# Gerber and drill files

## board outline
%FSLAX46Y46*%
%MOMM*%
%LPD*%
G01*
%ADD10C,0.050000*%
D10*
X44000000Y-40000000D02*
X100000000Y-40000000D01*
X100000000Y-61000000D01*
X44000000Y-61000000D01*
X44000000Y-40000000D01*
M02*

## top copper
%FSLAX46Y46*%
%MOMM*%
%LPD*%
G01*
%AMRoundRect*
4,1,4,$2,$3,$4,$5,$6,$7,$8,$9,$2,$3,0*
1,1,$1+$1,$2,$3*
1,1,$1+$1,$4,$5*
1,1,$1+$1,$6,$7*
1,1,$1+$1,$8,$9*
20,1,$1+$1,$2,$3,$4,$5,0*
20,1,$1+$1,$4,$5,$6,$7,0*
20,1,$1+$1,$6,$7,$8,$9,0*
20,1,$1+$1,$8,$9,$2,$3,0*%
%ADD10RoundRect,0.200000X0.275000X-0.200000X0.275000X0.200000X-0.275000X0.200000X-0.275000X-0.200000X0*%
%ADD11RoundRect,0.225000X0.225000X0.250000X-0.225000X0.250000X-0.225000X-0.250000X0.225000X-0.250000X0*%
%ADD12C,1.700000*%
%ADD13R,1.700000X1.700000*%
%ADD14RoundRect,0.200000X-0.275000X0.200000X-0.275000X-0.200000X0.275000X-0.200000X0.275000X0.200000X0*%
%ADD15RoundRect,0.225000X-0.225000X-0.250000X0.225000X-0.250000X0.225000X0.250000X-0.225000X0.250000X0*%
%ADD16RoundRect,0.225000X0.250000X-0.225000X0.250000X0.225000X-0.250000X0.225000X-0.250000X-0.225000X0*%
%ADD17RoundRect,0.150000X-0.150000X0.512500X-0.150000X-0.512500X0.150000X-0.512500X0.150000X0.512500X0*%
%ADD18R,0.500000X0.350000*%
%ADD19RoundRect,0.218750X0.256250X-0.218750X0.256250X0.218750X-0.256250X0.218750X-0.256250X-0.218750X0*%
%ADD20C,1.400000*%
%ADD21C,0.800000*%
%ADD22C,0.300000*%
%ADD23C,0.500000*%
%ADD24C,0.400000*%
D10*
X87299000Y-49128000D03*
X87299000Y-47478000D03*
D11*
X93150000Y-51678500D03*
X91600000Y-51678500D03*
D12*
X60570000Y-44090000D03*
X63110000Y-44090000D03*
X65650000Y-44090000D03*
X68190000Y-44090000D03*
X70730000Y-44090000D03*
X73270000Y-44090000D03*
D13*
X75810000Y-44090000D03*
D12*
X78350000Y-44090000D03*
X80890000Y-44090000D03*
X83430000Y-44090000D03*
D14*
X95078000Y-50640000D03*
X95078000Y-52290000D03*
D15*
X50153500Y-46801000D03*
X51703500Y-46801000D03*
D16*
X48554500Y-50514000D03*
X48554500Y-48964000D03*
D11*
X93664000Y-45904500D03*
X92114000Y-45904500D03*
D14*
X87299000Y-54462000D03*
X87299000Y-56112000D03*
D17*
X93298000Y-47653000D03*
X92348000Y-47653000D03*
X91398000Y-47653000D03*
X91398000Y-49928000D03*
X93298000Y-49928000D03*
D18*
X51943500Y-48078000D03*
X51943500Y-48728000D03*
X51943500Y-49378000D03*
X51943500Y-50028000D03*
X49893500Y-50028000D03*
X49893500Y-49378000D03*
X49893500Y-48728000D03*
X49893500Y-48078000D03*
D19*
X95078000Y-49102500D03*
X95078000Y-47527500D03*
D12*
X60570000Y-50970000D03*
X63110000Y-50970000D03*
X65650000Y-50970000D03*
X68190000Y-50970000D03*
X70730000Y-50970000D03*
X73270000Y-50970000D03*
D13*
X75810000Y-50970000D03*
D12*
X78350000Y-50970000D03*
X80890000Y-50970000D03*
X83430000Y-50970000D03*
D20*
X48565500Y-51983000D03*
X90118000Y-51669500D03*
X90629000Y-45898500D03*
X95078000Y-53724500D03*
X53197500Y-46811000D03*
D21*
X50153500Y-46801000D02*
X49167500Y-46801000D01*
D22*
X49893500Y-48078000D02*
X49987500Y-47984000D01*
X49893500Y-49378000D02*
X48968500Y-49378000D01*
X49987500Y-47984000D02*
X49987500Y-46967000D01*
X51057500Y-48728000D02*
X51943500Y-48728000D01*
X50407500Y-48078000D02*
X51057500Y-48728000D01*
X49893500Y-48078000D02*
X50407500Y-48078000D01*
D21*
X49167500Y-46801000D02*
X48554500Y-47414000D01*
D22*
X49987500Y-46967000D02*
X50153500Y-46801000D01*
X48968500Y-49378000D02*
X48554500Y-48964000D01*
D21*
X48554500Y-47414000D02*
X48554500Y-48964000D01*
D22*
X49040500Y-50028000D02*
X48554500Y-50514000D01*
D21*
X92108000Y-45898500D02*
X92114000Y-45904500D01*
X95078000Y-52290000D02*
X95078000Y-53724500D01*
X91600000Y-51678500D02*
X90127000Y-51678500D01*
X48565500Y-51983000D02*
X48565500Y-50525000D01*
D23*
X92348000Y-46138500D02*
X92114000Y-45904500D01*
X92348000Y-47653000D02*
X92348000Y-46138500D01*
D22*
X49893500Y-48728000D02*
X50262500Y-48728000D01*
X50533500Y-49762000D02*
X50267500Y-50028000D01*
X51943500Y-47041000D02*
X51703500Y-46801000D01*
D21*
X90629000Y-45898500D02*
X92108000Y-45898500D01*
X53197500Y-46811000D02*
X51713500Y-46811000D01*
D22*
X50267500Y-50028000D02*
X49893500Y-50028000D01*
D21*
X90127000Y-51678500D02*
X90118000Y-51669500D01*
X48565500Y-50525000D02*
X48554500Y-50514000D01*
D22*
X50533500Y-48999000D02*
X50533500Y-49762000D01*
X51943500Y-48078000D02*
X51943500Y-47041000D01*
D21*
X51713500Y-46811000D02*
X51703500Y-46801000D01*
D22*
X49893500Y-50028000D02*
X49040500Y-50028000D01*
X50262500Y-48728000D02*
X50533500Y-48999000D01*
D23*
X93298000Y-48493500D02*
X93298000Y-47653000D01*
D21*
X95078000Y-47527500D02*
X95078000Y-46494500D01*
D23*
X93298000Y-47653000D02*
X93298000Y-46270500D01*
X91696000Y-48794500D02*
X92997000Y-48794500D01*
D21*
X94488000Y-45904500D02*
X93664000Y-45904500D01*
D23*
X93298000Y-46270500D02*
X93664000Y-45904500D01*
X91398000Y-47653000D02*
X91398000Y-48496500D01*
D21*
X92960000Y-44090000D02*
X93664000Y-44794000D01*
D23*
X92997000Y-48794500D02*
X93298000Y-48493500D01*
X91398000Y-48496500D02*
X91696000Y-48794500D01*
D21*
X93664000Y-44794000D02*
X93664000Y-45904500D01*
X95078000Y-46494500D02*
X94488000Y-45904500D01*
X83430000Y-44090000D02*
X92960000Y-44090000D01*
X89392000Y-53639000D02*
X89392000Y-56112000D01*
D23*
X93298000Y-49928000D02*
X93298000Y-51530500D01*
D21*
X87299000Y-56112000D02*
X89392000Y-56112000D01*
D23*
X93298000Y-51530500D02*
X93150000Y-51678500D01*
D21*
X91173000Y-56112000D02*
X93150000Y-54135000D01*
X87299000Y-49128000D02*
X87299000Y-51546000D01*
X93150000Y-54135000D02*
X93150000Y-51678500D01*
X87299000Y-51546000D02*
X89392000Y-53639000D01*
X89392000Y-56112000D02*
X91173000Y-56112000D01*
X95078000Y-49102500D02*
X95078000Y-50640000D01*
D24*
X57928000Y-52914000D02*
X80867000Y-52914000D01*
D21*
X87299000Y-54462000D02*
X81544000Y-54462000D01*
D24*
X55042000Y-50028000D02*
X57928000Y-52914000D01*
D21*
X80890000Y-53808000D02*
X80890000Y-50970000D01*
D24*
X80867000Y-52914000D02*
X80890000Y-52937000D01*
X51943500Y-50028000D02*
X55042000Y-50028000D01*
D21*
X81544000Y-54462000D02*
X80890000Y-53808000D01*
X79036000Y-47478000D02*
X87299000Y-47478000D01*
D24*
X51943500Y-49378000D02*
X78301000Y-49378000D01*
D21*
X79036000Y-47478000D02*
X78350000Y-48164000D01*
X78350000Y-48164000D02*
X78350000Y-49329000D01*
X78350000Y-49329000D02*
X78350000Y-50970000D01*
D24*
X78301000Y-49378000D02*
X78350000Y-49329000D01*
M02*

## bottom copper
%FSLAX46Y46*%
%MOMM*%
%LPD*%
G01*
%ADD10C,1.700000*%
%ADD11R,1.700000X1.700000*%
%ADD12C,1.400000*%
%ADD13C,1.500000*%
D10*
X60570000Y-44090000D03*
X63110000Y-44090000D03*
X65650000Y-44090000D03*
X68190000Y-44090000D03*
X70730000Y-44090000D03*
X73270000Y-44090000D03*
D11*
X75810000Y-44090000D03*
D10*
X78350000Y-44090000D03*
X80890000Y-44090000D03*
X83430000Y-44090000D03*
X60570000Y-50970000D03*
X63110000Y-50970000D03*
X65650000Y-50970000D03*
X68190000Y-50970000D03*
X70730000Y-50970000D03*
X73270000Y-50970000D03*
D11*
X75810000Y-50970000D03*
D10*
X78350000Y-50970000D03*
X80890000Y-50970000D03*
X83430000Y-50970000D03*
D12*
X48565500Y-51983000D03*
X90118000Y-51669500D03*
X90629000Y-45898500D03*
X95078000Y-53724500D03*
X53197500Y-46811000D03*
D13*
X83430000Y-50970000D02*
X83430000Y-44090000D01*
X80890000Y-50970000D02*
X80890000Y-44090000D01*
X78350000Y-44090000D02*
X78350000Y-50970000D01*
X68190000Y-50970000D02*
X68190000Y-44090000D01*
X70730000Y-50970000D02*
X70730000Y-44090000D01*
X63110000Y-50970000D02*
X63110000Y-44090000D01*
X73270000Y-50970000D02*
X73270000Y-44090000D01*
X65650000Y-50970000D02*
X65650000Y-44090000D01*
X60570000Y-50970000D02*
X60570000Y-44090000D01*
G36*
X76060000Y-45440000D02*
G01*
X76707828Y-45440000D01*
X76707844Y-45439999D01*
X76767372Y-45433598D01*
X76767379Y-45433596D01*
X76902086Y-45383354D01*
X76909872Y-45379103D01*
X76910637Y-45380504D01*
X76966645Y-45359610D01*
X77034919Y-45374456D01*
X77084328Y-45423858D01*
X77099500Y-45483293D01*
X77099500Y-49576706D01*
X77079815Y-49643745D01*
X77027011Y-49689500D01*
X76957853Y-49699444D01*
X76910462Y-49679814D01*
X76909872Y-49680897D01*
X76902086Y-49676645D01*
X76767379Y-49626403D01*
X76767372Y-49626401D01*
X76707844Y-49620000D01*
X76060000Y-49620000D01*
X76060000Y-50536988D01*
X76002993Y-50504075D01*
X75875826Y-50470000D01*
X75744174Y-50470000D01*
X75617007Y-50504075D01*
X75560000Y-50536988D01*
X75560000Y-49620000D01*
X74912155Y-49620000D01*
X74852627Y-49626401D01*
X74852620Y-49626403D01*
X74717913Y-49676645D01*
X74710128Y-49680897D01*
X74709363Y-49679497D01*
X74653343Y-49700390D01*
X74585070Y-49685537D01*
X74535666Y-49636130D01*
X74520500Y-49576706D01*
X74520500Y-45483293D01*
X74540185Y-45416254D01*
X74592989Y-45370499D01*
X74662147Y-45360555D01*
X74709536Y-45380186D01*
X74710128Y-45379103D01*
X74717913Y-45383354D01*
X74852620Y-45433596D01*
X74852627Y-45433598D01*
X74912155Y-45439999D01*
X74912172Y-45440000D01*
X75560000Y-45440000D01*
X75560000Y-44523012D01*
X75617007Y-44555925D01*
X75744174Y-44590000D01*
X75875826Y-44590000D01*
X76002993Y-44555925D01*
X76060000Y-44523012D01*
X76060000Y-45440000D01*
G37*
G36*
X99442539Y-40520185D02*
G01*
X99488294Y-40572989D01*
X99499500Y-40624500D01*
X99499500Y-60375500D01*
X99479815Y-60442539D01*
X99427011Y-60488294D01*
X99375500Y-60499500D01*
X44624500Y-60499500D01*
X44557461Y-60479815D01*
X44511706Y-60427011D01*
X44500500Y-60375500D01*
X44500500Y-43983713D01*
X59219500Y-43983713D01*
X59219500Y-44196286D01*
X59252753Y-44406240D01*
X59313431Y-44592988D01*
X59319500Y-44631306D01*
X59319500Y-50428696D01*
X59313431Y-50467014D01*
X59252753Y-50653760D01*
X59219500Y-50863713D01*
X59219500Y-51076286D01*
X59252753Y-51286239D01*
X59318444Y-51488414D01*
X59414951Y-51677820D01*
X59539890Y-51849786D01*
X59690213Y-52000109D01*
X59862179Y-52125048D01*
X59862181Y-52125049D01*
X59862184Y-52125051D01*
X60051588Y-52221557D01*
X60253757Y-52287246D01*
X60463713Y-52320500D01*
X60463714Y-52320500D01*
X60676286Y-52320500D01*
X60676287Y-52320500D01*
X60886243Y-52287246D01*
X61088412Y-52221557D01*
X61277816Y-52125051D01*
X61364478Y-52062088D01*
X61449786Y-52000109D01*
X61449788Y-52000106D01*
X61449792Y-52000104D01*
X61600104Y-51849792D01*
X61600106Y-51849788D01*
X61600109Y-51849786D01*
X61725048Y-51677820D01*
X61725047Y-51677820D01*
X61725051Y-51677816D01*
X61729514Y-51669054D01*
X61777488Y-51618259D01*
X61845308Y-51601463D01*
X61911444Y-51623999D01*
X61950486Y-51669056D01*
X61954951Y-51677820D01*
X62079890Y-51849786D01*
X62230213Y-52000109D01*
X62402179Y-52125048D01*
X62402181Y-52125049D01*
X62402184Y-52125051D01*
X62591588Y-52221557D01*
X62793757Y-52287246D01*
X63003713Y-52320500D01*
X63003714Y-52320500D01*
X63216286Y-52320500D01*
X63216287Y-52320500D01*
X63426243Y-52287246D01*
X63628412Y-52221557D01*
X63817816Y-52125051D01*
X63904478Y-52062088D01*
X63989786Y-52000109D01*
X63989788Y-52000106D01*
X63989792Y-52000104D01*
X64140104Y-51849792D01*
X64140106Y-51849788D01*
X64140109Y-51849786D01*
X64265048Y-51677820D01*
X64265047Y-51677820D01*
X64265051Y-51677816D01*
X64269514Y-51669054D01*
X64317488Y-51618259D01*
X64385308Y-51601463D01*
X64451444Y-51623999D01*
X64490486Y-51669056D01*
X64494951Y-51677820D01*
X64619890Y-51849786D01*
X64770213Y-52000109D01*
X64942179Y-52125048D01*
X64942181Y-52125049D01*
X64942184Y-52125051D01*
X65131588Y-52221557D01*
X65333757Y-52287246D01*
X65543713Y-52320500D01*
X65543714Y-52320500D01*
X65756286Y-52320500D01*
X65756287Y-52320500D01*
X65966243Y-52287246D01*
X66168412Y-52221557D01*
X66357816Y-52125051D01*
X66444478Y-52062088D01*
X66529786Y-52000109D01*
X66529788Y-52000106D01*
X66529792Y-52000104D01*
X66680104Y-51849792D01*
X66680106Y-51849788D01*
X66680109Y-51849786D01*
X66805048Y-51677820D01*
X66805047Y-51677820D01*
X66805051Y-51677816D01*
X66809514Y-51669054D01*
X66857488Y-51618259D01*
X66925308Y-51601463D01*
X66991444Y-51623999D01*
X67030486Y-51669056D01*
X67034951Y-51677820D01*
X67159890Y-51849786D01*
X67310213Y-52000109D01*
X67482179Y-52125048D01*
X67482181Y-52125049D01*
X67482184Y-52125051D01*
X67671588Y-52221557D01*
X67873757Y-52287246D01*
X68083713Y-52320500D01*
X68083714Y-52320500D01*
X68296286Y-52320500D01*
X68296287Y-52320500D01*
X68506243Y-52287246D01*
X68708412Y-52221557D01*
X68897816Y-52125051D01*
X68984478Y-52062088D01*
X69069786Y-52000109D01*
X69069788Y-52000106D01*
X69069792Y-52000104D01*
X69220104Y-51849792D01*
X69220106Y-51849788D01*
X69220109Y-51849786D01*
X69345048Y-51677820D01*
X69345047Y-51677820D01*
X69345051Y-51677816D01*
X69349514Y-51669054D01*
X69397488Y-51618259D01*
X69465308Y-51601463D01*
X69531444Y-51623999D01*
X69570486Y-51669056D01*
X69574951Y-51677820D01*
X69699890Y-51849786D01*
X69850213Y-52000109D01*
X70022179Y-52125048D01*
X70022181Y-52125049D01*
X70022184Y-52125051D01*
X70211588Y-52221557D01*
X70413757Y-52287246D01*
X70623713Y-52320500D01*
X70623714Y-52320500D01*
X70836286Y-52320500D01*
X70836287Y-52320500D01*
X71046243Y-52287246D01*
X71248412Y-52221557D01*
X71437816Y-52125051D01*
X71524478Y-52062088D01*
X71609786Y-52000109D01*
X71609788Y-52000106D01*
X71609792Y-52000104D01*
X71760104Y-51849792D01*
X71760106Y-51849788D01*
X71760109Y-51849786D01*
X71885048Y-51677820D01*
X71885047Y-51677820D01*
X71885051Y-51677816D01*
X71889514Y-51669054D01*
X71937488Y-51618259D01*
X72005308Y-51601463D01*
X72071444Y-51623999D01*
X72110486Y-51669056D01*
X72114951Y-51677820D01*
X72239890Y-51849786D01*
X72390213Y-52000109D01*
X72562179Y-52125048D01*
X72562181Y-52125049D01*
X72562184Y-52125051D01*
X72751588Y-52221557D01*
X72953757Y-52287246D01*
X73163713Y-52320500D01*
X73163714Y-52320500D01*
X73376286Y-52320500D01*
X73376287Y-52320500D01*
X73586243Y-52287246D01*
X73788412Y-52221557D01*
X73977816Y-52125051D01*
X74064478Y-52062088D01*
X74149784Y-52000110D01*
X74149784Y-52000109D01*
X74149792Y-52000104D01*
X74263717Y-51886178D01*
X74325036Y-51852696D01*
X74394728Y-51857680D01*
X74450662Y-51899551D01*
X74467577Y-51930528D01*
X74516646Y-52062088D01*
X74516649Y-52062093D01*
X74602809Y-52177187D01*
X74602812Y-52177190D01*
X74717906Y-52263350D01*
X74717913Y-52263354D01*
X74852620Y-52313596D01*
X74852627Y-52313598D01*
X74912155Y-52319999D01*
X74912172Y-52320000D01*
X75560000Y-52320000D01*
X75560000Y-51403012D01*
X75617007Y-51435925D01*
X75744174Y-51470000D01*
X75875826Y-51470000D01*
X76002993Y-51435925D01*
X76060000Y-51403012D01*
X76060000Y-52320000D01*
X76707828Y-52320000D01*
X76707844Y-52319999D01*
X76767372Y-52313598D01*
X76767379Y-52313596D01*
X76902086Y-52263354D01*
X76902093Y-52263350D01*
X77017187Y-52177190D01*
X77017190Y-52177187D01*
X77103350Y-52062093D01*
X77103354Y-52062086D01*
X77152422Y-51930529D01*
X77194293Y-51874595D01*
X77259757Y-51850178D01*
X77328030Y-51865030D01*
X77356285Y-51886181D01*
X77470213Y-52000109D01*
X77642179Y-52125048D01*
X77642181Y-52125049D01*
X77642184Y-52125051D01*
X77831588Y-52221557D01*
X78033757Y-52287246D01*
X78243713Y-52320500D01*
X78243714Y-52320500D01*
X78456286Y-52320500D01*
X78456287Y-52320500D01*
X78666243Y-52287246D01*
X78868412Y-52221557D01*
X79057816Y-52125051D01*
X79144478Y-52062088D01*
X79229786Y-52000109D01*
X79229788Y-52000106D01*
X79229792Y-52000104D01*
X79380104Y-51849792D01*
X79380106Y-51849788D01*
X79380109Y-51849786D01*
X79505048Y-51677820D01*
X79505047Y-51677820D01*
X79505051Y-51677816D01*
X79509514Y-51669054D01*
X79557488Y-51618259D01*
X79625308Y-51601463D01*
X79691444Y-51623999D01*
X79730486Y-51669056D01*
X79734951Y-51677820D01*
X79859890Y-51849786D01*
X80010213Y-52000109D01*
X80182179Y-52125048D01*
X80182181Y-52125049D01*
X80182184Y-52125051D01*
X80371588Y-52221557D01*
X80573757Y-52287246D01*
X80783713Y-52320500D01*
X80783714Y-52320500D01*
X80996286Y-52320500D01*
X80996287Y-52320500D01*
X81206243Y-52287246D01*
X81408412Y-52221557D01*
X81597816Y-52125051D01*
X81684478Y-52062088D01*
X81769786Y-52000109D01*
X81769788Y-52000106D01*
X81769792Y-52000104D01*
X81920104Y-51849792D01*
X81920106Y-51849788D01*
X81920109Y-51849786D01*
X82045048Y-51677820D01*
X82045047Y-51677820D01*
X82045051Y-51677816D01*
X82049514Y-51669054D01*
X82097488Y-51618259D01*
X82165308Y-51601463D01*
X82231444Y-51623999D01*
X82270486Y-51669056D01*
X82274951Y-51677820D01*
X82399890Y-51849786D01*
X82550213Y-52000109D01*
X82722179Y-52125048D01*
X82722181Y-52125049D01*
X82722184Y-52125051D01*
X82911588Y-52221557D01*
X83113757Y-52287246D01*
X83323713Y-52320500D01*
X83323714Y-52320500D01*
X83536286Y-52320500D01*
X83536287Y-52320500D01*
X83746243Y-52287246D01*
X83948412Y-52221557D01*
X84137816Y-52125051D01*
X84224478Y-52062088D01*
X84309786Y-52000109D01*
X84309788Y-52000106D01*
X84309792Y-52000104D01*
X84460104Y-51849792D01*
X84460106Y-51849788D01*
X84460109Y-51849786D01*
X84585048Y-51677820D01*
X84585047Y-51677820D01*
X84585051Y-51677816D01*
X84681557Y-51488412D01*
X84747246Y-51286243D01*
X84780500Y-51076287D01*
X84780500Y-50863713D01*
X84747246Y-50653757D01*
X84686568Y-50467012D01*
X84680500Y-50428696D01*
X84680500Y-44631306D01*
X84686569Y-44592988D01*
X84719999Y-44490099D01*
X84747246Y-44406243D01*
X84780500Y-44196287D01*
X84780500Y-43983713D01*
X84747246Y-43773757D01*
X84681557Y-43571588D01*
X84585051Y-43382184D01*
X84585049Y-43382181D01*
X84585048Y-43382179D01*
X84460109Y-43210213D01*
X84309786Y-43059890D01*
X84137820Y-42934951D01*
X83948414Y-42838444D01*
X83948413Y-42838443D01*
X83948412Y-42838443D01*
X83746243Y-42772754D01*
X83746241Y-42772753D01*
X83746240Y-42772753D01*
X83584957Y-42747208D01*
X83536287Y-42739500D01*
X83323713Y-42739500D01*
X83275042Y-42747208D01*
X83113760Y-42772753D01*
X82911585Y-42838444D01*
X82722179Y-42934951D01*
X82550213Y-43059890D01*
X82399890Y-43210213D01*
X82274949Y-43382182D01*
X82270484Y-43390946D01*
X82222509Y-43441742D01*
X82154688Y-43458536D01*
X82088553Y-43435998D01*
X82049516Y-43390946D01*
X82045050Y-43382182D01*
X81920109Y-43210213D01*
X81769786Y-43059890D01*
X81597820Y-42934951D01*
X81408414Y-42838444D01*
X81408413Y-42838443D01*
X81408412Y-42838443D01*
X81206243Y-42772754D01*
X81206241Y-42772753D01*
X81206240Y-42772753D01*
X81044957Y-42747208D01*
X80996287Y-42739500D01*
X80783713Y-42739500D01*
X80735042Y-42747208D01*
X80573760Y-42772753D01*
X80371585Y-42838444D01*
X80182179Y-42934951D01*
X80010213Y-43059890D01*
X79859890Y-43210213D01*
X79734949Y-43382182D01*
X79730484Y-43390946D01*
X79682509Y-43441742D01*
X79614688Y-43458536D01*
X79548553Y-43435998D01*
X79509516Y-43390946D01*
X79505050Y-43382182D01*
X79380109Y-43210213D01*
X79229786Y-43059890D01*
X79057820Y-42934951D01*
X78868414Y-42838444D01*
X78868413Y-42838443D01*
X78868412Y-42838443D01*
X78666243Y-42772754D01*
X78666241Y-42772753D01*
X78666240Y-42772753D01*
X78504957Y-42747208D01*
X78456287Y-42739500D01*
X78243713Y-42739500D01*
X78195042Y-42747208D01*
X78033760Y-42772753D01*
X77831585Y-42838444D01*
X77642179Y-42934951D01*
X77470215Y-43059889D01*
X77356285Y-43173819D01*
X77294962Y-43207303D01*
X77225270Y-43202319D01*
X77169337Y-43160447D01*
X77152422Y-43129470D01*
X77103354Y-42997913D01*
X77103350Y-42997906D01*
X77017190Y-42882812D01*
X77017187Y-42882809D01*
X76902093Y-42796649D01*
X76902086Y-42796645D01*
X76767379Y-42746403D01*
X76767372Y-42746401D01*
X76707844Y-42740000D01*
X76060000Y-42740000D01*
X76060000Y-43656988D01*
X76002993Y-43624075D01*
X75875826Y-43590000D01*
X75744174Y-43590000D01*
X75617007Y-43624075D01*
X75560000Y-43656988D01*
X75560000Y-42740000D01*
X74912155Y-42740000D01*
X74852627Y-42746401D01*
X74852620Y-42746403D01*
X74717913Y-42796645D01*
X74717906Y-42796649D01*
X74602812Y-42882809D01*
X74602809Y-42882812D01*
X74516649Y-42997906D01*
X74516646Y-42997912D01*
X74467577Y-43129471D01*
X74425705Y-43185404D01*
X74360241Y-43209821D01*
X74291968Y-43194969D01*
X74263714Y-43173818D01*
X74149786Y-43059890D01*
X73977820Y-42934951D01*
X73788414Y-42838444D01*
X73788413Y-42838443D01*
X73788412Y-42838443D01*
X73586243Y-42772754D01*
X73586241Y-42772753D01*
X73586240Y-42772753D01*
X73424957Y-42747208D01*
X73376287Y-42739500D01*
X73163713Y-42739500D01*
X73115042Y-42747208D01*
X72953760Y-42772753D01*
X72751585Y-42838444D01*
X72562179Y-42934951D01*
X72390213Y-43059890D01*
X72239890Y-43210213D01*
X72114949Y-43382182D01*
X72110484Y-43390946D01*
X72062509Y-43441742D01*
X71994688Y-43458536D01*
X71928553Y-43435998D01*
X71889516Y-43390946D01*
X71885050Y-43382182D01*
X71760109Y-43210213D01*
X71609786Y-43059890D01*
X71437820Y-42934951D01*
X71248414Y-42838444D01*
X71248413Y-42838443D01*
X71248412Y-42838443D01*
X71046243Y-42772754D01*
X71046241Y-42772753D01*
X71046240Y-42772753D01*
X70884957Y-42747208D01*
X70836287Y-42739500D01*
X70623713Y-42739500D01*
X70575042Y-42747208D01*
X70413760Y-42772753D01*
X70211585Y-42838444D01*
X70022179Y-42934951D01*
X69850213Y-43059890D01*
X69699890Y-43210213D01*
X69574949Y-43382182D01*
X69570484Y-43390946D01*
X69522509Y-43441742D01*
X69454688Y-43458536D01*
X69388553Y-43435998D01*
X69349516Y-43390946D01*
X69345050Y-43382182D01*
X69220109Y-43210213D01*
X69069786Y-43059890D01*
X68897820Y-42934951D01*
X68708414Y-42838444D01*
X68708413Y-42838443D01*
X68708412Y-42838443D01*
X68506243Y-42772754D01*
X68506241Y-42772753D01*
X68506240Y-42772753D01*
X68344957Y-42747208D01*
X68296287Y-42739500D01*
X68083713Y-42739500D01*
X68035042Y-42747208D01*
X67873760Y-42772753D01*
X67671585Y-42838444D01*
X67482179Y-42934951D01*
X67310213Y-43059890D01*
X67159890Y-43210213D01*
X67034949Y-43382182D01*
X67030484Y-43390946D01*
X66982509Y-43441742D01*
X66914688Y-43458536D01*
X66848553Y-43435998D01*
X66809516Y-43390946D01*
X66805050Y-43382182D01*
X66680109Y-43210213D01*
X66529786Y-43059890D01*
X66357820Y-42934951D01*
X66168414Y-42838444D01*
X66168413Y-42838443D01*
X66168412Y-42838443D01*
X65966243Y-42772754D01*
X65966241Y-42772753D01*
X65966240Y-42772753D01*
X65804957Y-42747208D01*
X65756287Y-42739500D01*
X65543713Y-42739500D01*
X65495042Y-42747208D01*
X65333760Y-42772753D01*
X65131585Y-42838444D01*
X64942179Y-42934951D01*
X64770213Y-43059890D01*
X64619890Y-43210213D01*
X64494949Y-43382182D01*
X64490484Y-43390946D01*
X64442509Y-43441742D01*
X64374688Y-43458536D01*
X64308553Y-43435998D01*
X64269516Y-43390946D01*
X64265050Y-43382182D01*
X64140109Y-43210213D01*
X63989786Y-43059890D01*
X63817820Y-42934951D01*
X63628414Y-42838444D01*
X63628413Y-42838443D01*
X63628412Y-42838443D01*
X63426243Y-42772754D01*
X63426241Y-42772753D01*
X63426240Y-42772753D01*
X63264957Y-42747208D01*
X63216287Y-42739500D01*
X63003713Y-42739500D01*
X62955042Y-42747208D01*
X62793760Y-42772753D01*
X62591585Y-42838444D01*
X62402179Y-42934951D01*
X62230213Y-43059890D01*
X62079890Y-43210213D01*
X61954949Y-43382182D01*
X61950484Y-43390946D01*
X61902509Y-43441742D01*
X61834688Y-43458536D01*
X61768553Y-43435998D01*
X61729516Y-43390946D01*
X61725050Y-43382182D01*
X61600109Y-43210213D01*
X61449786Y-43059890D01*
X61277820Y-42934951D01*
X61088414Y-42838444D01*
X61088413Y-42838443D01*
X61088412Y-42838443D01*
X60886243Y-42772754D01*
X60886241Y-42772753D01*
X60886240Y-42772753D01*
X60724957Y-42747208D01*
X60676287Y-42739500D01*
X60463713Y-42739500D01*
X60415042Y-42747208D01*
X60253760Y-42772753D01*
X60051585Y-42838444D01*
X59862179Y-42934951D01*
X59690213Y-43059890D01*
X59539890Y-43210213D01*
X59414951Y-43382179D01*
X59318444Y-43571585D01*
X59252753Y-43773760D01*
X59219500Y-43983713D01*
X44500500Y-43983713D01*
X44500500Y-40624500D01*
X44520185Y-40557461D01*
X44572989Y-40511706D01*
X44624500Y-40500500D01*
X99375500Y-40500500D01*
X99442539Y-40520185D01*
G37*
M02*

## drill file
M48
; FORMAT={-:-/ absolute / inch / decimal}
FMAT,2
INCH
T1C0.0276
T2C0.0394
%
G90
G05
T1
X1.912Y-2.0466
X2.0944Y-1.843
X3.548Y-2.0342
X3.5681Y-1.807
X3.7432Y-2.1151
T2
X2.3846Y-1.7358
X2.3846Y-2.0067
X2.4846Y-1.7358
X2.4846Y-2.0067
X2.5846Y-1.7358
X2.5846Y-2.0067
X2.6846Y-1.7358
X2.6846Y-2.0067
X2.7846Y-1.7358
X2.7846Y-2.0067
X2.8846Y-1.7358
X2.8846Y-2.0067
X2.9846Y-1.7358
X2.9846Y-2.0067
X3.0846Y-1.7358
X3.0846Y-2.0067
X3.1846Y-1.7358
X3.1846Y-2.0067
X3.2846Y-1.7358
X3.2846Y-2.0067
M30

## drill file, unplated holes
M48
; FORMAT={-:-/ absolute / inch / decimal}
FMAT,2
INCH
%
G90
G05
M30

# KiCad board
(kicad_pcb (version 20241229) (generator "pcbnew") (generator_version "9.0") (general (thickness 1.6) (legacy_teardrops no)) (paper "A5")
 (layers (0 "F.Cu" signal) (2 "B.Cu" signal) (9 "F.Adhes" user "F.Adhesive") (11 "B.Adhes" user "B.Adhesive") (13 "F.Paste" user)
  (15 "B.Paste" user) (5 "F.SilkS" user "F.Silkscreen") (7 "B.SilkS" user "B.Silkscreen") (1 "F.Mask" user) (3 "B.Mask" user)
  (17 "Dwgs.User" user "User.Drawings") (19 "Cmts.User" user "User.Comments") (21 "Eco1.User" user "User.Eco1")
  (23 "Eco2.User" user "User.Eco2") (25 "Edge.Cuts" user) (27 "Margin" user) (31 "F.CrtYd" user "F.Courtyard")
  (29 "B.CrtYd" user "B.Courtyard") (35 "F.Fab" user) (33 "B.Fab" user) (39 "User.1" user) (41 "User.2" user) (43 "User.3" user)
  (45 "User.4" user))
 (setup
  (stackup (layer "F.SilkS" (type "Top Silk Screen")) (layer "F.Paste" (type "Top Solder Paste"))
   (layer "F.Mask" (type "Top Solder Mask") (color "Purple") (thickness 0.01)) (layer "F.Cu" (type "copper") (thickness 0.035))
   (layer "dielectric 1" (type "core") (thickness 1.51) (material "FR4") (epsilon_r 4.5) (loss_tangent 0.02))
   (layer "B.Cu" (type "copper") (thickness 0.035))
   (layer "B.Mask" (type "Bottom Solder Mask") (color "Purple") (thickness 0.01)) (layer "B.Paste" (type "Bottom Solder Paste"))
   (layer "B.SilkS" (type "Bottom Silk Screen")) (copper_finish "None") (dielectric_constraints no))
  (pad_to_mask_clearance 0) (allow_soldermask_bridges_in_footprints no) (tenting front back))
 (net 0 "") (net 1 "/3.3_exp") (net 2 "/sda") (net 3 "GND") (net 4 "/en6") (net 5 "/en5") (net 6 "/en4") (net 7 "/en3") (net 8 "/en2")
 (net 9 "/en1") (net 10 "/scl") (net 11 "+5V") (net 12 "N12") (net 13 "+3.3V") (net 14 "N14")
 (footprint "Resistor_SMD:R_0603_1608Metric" (layer "F.Cu") (at 87.299 48.303 90)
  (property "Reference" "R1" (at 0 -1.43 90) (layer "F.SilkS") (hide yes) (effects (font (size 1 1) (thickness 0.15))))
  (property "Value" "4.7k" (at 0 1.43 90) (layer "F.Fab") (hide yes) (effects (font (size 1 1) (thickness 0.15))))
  (pad "1" smd roundrect (at -0.825 0 90) (size 0.8 0.95) (layers "F.Cu" "F.Mask" "F.Paste") (roundrect_rratio 0.25) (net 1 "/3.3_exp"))
  (pad "2" smd roundrect (at 0.825 0 90) (size 0.8 0.95) (layers "F.Cu" "F.Mask" "F.Paste") (roundrect_rratio 0.25) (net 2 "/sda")))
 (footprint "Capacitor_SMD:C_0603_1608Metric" (layer "F.Cu") (at 92.375 51.6785 180)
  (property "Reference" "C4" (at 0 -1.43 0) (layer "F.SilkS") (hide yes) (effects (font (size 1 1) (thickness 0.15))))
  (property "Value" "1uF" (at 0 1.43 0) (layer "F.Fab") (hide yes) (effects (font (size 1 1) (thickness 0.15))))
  (pad "1" smd roundrect (at -0.775 0 180) (size 0.9 0.95) (layers "F.Cu" "F.Mask" "F.Paste") (roundrect_rratio 0.25) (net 1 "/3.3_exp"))
  (pad "2" smd roundrect (at 0.775 0 180) (size 0.9 0.95) (layers "F.Cu" "F.Mask" "F.Paste") (roundrect_rratio 0.25) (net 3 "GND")))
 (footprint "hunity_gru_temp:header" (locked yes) (layer "F.Cu") (at 60.57 44.09 90)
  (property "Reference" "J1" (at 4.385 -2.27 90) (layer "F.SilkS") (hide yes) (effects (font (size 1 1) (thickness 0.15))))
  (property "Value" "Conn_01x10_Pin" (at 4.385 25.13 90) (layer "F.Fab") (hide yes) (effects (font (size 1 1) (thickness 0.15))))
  (pad "1" thru_hole circle (at 0 0 90) (size 1.7 1.7) (drill 1) (layers "*.Cu" "*.Mask") (remove_unused_layers no) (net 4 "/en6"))
  (pad "2" thru_hole circle (at 0 2.54 90) (size 1.7 1.7) (drill 1) (layers "*.Cu" "*.Mask") (remove_unused_layers no) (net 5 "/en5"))
  (pad "3" thru_hole circle (at 0 5.08 90) (size 1.7 1.7) (drill 1) (layers "*.Cu" "*.Mask") (remove_unused_layers no) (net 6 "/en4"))
  (pad "4" thru_hole circle (at 0 7.62 90) (size 1.7 1.7) (drill 1) (layers "*.Cu" "*.Mask") (remove_unused_layers no) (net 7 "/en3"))
  (pad "5" thru_hole circle (at 0 10.16 90) (size 1.7 1.7) (drill 1) (layers "*.Cu" "*.Mask") (remove_unused_layers no) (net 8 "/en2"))
  (pad "6" thru_hole circle (at 0 12.7 90) (size 1.7 1.7) (drill 1) (layers "*.Cu" "*.Mask") (remove_unused_layers no) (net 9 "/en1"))
  (pad "7" thru_hole rect (at 0 15.24 90) (size 1.7 1.7) (drill 1) (layers "*.Cu" "*.Mask") (remove_unused_layers no) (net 3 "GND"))
  (pad "8" thru_hole circle (at 0 17.78 90) (size 1.7 1.7) (drill 1) (layers "*.Cu" "*.Mask") (remove_unused_layers no) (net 2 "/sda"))
  (pad "9" thru_hole circle (at 0 20.32 90) (size 1.7 1.7) (drill 1) (layers "*.Cu" "*.Mask") (remove_unused_layers no) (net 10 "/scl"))
  (pad "10" thru_hole circle (at 0 22.86 90) (size 1.7 1.7) (drill 1) (layers "*.Cu" "*.Mask") (remove_unused_layers no) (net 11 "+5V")))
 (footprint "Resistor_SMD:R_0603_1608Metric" (layer "F.Cu") (at 95.078 51.465 -90)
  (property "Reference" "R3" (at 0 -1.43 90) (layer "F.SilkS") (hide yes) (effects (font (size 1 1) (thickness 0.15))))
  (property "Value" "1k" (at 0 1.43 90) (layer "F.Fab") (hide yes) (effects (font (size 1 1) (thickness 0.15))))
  (pad "1" smd roundrect (at -0.825 0 270) (size 0.8 0.95) (layers "F.Cu" "F.Mask" "F.Paste") (roundrect_rratio 0.25) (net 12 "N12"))
  (pad "2" smd roundrect (at 0.825 0 270) (size 0.8 0.95) (layers "F.Cu" "F.Mask" "F.Paste") (roundrect_rratio 0.25) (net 3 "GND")))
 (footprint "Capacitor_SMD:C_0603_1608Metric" (layer "F.Cu") (at 50.9285 46.801)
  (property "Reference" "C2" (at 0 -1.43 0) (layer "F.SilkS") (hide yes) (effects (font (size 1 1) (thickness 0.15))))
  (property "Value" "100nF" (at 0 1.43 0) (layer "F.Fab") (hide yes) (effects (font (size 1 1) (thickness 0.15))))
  (pad "1" smd roundrect (at -0.775 0) (size 0.9 0.95) (layers "F.Cu" "F.Mask" "F.Paste") (roundrect_rratio 0.25) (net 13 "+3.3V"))
  (pad "2" smd roundrect (at 0.775 0) (size 0.9 0.95) (layers "F.Cu" "F.Mask" "F.Paste") (roundrect_rratio 0.25) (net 3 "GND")))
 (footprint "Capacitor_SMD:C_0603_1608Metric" (layer "F.Cu") (at 48.5545 49.739 90)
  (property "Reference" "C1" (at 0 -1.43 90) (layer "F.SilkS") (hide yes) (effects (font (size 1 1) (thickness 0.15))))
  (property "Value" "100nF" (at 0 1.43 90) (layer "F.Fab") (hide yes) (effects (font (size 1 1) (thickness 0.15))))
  (pad "1" smd roundrect (at -0.775 0 90) (size 0.9 0.95) (layers "F.Cu" "F.Mask" "F.Paste") (roundrect_rratio 0.25) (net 3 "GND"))
  (pad "2" smd roundrect (at 0.775 0 90) (size 0.9 0.95) (layers "F.Cu" "F.Mask" "F.Paste") (roundrect_rratio 0.25) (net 13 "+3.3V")))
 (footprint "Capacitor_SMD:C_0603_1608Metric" (layer "F.Cu") (at 92.889 45.9045 180)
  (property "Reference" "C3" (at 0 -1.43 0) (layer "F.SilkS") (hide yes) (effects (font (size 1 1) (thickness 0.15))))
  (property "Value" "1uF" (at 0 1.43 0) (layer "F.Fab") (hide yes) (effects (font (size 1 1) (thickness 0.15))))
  (pad "1" smd roundrect (at -0.775 0 180) (size 0.9 0.95) (layers "F.Cu" "F.Mask" "F.Paste") (roundrect_rratio 0.25) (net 11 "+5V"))
  (pad "2" smd roundrect (at 0.775 0 180) (size 0.9 0.95) (layers "F.Cu" "F.Mask" "F.Paste") (roundrect_rratio 0.25) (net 3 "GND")))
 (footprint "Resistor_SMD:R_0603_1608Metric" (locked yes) (layer "F.Cu") (at 87.299 55.287 -90)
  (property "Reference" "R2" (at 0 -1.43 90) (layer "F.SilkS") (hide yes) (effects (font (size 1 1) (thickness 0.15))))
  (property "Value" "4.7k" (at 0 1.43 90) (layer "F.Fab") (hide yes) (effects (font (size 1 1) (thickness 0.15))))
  (pad "1" smd roundrect (at -0.825 0 270) (size 0.8 0.95) (layers "F.Cu" "F.Mask" "F.Paste") (roundrect_rratio 0.25) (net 10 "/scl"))
  (pad "2" smd roundrect (at 0.825 0 270) (size 0.8 0.95) (layers "F.Cu" "F.Mask" "F.Paste") (roundrect_rratio 0.25) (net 1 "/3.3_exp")))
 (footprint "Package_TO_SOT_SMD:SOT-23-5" (layer "F.Cu") (at 92.348 48.7905 -90)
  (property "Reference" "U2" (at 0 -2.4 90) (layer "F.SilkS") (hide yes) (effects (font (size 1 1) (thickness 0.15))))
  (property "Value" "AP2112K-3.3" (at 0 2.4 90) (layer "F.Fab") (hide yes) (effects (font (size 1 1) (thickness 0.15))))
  (pad "1" smd roundrect (at -1.1375 -0.95 270) (size 1.325 0.6) (layers "F.Cu" "F.Mask" "F.Paste") (roundrect_rratio 0.25) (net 11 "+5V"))
  (pad "2" smd roundrect (at -1.1375 0 270) (size 1.325 0.6) (layers "F.Cu" "F.Mask" "F.Paste") (roundrect_rratio 0.25) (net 3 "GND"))
  (pad "3" smd roundrect (at -1.1375 0.95 270) (size 1.325 0.6) (layers "F.Cu" "F.Mask" "F.Paste") (roundrect_rratio 0.25) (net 11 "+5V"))
  (pad "4" smd roundrect (at 1.1375 0.95 270) (size 1.325 0.6) (layers "F.Cu" "F.Mask" "F.Paste") (roundrect_rratio 0.25) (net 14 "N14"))
  (pad "5" smd roundrect (at 1.1375 -0.95 270) (size 1.325 0.6) (layers "F.Cu" "F.Mask" "F.Paste") (roundrect_rratio 0.25)
   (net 1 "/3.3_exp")))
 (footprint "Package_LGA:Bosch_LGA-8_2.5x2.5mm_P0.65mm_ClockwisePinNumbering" (layer "F.Cu") (at 50.9185 49.053 -90)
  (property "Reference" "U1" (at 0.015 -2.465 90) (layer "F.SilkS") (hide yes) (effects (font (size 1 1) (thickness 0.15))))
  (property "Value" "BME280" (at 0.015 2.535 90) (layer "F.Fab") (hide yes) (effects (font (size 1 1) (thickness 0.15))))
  (pad "1" smd rect (at -0.975 -1.025) (size 0.5 0.35) (layers "F.Cu" "F.Mask" "F.Paste") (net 3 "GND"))
  (pad "2" smd rect (at -0.325 -1.025) (size 0.5 0.35) (layers "F.Cu" "F.Mask" "F.Paste") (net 13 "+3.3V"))
  (pad "3" smd rect (at 0.325 -1.025) (size 0.5 0.35) (layers "F.Cu" "F.Mask" "F.Paste") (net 2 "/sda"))
  (pad "4" smd rect (at 0.975 -1.025) (size 0.5 0.35) (layers "F.Cu" "F.Mask" "F.Paste") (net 10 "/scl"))
  (pad "5" smd rect (at 0.975 1.025) (size 0.5 0.35) (layers "F.Cu" "F.Mask" "F.Paste") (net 3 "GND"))
  (pad "6" smd rect (at 0.325 1.025) (size 0.5 0.35) (layers "F.Cu" "F.Mask" "F.Paste") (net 13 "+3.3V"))
  (pad "7" smd rect (at -0.325 1.025) (size 0.5 0.35) (layers "F.Cu" "F.Mask" "F.Paste") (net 3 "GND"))
  (pad "8" smd rect (at -0.975 1.025) (size 0.5 0.35) (layers "F.Cu" "F.Mask" "F.Paste") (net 13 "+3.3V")))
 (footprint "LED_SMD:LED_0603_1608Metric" (layer "F.Cu") (at 95.078 48.315 90)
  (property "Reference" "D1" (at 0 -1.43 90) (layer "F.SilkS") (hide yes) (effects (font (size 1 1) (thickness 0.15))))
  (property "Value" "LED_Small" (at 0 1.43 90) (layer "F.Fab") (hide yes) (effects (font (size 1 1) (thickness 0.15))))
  (pad "1" smd roundrect (at -0.7875 0 90) (size 0.875 0.95) (layers "F.Cu" "F.Mask" "F.Paste") (roundrect_rratio 0.25) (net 12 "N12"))
  (pad "2" smd roundrect (at 0.7875 0 90) (size 0.875 0.95) (layers "F.Cu" "F.Mask" "F.Paste") (roundrect_rratio 0.25) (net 11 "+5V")))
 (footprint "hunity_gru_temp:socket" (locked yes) (layer "F.Cu") (at 60.57 50.97 90)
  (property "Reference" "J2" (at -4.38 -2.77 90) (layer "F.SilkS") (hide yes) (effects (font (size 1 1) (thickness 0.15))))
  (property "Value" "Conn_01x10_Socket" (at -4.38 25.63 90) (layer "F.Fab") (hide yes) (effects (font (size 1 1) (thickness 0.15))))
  (pad "1" thru_hole circle (at 0 0 90) (size 1.7 1.7) (drill 1) (layers "*.Cu" "*.Mask") (remove_unused_layers no) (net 4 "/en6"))
  (pad "2" thru_hole circle (at 0 2.54 90) (size 1.7 1.7) (drill 1) (layers "*.Cu" "*.Mask") (remove_unused_layers no) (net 5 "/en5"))
  (pad "3" thru_hole circle (at 0 5.08 90) (size 1.7 1.7) (drill 1) (layers "*.Cu" "*.Mask") (remove_unused_layers no) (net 6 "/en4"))
  (pad "4" thru_hole circle (at 0 7.62 90) (size 1.7 1.7) (drill 1) (layers "*.Cu" "*.Mask") (remove_unused_layers no) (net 7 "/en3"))
  (pad "5" thru_hole circle (at 0 10.16 90) (size 1.7 1.7) (drill 1) (layers "*.Cu" "*.Mask") (remove_unused_layers no) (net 8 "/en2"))
  (pad "6" thru_hole circle (at 0 12.7 90) (size 1.7 1.7) (drill 1) (layers "*.Cu" "*.Mask") (remove_unused_layers no) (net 9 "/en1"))
  (pad "7" thru_hole rect (at 0 15.24 90) (size 1.7 1.7) (drill 1) (layers "*.Cu" "*.Mask") (remove_unused_layers no) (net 3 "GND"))
  (pad "8" thru_hole circle (at 0 17.78 90) (size 1.7 1.7) (drill 1) (layers "*.Cu" "*.Mask") (remove_unused_layers no) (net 2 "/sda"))
  (pad "9" thru_hole circle (at 0 20.32 90) (size 1.7 1.7) (drill 1) (layers "*.Cu" "*.Mask") (remove_unused_layers no) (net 10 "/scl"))
  (pad "10" thru_hole circle (at 0 22.86 90) (size 1.7 1.7) (drill 1) (layers "*.Cu" "*.Mask") (remove_unused_layers no) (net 11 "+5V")))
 (gr_rect (start 44 40) (end 100 61) (stroke (width 0.05) (type solid)) (fill no) (locked yes) (layer "Edge.Cuts"))
 (segment (start 50.1535 46.801) (end 49.1675 46.801) (width 0.8) (layer "F.Cu") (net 13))
 (segment (start 49.8935 48.078) (end 49.9875 47.984) (width 0.3) (layer "F.Cu") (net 13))
 (segment (start 49.8935 49.378) (end 48.9685 49.378) (width 0.3) (layer "F.Cu") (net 13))
 (segment (start 49.9875 47.984) (end 49.9875 46.967) (width 0.3) (layer "F.Cu") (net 13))
 (segment (start 51.0575 48.728) (end 51.9435 48.728) (width 0.3) (layer "F.Cu") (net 13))
 (segment (start 50.4075 48.078) (end 51.0575 48.728) (width 0.3) (layer "F.Cu") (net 13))
 (segment (start 49.8935 48.078) (end 50.4075 48.078) (width 0.3) (layer "F.Cu") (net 13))
 (segment (start 49.1675 46.801) (end 48.5545 47.414) (width 0.8) (layer "F.Cu") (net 13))
 (segment (start 49.9875 46.967) (end 50.1535 46.801) (width 0.3) (layer "F.Cu") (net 13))
 (segment (start 48.9685 49.378) (end 48.5545 48.964) (width 0.3) (layer "F.Cu") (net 13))
 (segment (start 48.5545 47.414) (end 48.5545 48.964) (width 0.8) (layer "F.Cu") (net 13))
 (segment (start 49.0405 50.028) (end 48.5545 50.514) (width 0.3) (layer "F.Cu") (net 3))
 (segment (start 92.108 45.8985) (end 92.114 45.9045) (width 0.8) (layer "F.Cu") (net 3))
 (segment (start 95.078 52.29) (end 95.078 53.7245) (width 0.8) (layer "F.Cu") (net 3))
 (segment (start 91.6 51.6785) (end 90.127 51.6785) (width 0.8) (layer "F.Cu") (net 3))
 (segment (start 48.5655 51.983) (end 48.5655 50.525) (width 0.8) (layer "F.Cu") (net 3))
 (segment (start 92.348 46.1385) (end 92.114 45.9045) (width 0.5) (layer "F.Cu") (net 3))
 (segment (start 92.348 47.653) (end 92.348 46.1385) (width 0.5) (layer "F.Cu") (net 3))
 (segment (start 49.8935 48.728) (end 50.2625 48.728) (width 0.3) (layer "F.Cu") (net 3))
 (segment (start 50.5335 49.762) (end 50.2675 50.028) (width 0.3) (layer "F.Cu") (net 3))
 (segment (start 51.9435 47.041) (end 51.7035 46.801) (width 0.3) (layer "F.Cu") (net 3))
 (segment (start 90.629 45.8985) (end 92.108 45.8985) (width 0.8) (layer "F.Cu") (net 3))
 (segment (start 53.1975 46.811) (end 51.7135 46.811) (width 0.8) (layer "F.Cu") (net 3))
 (segment (start 50.2675 50.028) (end 49.8935 50.028) (width 0.3) (layer "F.Cu") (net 3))
 (segment (start 90.127 51.6785) (end 90.118 51.6695) (width 0.8) (layer "F.Cu") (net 3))
 (segment (start 48.5655 50.525) (end 48.5545 50.514) (width 0.8) (layer "F.Cu") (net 3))
 (segment (start 50.5335 48.999) (end 50.5335 49.762) (width 0.3) (layer "F.Cu") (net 3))
 (segment (start 51.9435 48.078) (end 51.9435 47.041) (width 0.3) (layer "F.Cu") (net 3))
 (segment (start 51.7135 46.811) (end 51.7035 46.801) (width 0.8) (layer "F.Cu") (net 3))
 (segment (start 49.8935 50.028) (end 49.0405 50.028) (width 0.3) (layer "F.Cu") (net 3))
 (segment (start 50.2625 48.728) (end 50.5335 48.999) (width 0.3) (layer "F.Cu") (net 3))
 (via (at 48.5655 51.983) (size 1.4) (drill 0.7) (layers "F.Cu" "B.Cu") (free yes) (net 3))
 (via (at 90.118 51.6695) (size 1.4) (drill 0.7) (layers "F.Cu" "B.Cu") (free yes) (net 3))
 (via (at 90.629 45.8985) (size 1.4) (drill 0.7) (layers "F.Cu" "B.Cu") (free yes) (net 3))
 (via (at 95.078 53.7245) (size 1.4) (drill 0.7) (layers "F.Cu" "B.Cu") (free yes) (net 3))
 (via (at 53.1975 46.811) (size 1.4) (drill 0.7) (layers "F.Cu" "B.Cu") (free yes) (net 3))
 (segment (start 93.298 48.4935) (end 93.298 47.653) (width 0.5) (layer "F.Cu") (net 11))
 (segment (start 95.078 47.5275) (end 95.078 46.4945) (width 0.8) (layer "F.Cu") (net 11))
 (segment (start 93.298 47.653) (end 93.298 46.2705) (width 0.5) (layer "F.Cu") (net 11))
 (segment (start 91.696 48.7945) (end 92.997 48.7945) (width 0.5) (layer "F.Cu") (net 11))
 (segment (start 94.488 45.9045) (end 93.664 45.9045) (width 0.8) (layer "F.Cu") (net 11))
 (segment (start 93.298 46.2705) (end 93.664 45.9045) (width 0.5) (layer "F.Cu") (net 11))
 (segment (start 91.398 47.653) (end 91.398 48.4965) (width 0.5) (layer "F.Cu") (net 11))
 (segment (start 92.96 44.09) (end 93.664 44.794) (width 0.8) (layer "F.Cu") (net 11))
 (segment (start 92.997 48.7945) (end 93.298 48.4935) (width 0.5) (layer "F.Cu") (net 11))
 (segment (start 91.398 48.4965) (end 91.696 48.7945) (width 0.5) (layer "F.Cu") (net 11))
 (segment (start 93.664 44.794) (end 93.664 45.9045) (width 0.8) (layer "F.Cu") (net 11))
 (segment (start 95.078 46.4945) (end 94.488 45.9045) (width 0.8) (layer "F.Cu") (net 11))
 (segment (start 83.43 44.09) (end 92.96 44.09) (width 0.8) (layer "F.Cu") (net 11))
 (segment (start 83.43 50.97) (end 83.43 44.09) (width 1.5) (layer "B.Cu") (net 11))
 (segment (start 89.392 53.639) (end 89.392 56.112) (width 0.8) (layer "F.Cu") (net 1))
 (segment (start 93.298 49.928) (end 93.298 51.5305) (width 0.5) (layer "F.Cu") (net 1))
 (segment (start 87.299 56.112) (end 89.392 56.112) (width 0.8) (layer "F.Cu") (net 1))
 (segment (start 93.298 51.5305) (end 93.15 51.6785) (width 0.5) (layer "F.Cu") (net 1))
 (segment (start 91.173 56.112) (end 93.15 54.135) (width 0.8) (layer "F.Cu") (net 1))
 (segment (start 87.299 49.128) (end 87.299 51.546) (width 0.8) (layer "F.Cu") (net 1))
 (segment (start 93.15 54.135) (end 93.15 51.6785) (width 0.8) (layer "F.Cu") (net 1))
 (segment (start 87.299 51.546) (end 89.392 53.639) (width 0.8) (layer "F.Cu") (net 1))
 (segment (start 89.392 56.112) (end 91.173 56.112) (width 0.8) (layer "F.Cu") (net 1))
 (segment (start 95.078 49.1025) (end 95.078 50.64) (width 0.8) (layer "F.Cu") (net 12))
 (segment (start 57.928 52.914) (end 80.867 52.914) (width 0.4) (layer "F.Cu") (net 10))
 (segment (start 87.299 54.462) (end 81.544 54.462) (width 0.8) (layer "F.Cu") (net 10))
 (segment (start 55.042 50.028) (end 57.928 52.914) (width 0.4) (layer "F.Cu") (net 10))
 (segment (start 80.89 53.808) (end 80.89 50.97) (width 0.8) (layer "F.Cu") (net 10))
 (segment (start 80.867 52.914) (end 80.89 52.937) (width 0.4) (layer "F.Cu") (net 10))
 (segment (start 51.9435 50.028) (end 55.042 50.028) (width 0.4) (layer "F.Cu") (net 10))
 (segment (start 81.544 54.462) (end 80.89 53.808) (width 0.8) (layer "F.Cu") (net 10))
 (segment (start 80.89 50.97) (end 80.89 44.09) (width 1.5) (layer "B.Cu") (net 10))
 (segment (start 79.036 47.478) (end 87.299 47.478) (width 0.8) (layer "F.Cu") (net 2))
 (segment (start 51.9435 49.378) (end 78.301 49.378) (width 0.4) (layer "F.Cu") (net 2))
 (segment (start 79.036 47.478) (end 78.35 48.164) (width 0.8) (layer "F.Cu") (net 2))
 (segment (start 78.35 48.164) (end 78.35 49.329) (width 0.8) (layer "F.Cu") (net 2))
 (segment (start 78.35 49.329) (end 78.35 50.97) (width 0.8) (layer "F.Cu") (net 2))
 (segment (start 78.301 49.378) (end 78.35 49.329) (width 0.4) (layer "F.Cu") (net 2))
 (segment (start 78.35 44.09) (end 78.35 50.97) (width 1.5) (layer "B.Cu") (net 2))
 (segment (start 68.19 50.97) (end 68.19 44.09) (width 1.5) (layer "B.Cu") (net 7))
 (segment (start 70.73 50.97) (end 70.73 44.09) (width 1.5) (layer "B.Cu") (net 8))
 (segment (start 63.11 50.97) (end 63.11 44.09) (width 1.5) (layer "B.Cu") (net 5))
 (segment (start 73.27 50.97) (end 73.27 44.09) (width 1.5) (layer "B.Cu") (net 9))
 (segment (start 65.65 50.97) (end 65.65 44.09) (width 1.5) (layer "B.Cu") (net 6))
 (segment (start 60.57 50.97) (end 60.57 44.09) (width 1.5) (layer "B.Cu") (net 4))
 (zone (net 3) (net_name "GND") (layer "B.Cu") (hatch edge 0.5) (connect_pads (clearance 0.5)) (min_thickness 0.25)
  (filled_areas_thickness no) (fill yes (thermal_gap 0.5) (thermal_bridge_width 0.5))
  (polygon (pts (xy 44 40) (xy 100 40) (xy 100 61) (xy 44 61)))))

